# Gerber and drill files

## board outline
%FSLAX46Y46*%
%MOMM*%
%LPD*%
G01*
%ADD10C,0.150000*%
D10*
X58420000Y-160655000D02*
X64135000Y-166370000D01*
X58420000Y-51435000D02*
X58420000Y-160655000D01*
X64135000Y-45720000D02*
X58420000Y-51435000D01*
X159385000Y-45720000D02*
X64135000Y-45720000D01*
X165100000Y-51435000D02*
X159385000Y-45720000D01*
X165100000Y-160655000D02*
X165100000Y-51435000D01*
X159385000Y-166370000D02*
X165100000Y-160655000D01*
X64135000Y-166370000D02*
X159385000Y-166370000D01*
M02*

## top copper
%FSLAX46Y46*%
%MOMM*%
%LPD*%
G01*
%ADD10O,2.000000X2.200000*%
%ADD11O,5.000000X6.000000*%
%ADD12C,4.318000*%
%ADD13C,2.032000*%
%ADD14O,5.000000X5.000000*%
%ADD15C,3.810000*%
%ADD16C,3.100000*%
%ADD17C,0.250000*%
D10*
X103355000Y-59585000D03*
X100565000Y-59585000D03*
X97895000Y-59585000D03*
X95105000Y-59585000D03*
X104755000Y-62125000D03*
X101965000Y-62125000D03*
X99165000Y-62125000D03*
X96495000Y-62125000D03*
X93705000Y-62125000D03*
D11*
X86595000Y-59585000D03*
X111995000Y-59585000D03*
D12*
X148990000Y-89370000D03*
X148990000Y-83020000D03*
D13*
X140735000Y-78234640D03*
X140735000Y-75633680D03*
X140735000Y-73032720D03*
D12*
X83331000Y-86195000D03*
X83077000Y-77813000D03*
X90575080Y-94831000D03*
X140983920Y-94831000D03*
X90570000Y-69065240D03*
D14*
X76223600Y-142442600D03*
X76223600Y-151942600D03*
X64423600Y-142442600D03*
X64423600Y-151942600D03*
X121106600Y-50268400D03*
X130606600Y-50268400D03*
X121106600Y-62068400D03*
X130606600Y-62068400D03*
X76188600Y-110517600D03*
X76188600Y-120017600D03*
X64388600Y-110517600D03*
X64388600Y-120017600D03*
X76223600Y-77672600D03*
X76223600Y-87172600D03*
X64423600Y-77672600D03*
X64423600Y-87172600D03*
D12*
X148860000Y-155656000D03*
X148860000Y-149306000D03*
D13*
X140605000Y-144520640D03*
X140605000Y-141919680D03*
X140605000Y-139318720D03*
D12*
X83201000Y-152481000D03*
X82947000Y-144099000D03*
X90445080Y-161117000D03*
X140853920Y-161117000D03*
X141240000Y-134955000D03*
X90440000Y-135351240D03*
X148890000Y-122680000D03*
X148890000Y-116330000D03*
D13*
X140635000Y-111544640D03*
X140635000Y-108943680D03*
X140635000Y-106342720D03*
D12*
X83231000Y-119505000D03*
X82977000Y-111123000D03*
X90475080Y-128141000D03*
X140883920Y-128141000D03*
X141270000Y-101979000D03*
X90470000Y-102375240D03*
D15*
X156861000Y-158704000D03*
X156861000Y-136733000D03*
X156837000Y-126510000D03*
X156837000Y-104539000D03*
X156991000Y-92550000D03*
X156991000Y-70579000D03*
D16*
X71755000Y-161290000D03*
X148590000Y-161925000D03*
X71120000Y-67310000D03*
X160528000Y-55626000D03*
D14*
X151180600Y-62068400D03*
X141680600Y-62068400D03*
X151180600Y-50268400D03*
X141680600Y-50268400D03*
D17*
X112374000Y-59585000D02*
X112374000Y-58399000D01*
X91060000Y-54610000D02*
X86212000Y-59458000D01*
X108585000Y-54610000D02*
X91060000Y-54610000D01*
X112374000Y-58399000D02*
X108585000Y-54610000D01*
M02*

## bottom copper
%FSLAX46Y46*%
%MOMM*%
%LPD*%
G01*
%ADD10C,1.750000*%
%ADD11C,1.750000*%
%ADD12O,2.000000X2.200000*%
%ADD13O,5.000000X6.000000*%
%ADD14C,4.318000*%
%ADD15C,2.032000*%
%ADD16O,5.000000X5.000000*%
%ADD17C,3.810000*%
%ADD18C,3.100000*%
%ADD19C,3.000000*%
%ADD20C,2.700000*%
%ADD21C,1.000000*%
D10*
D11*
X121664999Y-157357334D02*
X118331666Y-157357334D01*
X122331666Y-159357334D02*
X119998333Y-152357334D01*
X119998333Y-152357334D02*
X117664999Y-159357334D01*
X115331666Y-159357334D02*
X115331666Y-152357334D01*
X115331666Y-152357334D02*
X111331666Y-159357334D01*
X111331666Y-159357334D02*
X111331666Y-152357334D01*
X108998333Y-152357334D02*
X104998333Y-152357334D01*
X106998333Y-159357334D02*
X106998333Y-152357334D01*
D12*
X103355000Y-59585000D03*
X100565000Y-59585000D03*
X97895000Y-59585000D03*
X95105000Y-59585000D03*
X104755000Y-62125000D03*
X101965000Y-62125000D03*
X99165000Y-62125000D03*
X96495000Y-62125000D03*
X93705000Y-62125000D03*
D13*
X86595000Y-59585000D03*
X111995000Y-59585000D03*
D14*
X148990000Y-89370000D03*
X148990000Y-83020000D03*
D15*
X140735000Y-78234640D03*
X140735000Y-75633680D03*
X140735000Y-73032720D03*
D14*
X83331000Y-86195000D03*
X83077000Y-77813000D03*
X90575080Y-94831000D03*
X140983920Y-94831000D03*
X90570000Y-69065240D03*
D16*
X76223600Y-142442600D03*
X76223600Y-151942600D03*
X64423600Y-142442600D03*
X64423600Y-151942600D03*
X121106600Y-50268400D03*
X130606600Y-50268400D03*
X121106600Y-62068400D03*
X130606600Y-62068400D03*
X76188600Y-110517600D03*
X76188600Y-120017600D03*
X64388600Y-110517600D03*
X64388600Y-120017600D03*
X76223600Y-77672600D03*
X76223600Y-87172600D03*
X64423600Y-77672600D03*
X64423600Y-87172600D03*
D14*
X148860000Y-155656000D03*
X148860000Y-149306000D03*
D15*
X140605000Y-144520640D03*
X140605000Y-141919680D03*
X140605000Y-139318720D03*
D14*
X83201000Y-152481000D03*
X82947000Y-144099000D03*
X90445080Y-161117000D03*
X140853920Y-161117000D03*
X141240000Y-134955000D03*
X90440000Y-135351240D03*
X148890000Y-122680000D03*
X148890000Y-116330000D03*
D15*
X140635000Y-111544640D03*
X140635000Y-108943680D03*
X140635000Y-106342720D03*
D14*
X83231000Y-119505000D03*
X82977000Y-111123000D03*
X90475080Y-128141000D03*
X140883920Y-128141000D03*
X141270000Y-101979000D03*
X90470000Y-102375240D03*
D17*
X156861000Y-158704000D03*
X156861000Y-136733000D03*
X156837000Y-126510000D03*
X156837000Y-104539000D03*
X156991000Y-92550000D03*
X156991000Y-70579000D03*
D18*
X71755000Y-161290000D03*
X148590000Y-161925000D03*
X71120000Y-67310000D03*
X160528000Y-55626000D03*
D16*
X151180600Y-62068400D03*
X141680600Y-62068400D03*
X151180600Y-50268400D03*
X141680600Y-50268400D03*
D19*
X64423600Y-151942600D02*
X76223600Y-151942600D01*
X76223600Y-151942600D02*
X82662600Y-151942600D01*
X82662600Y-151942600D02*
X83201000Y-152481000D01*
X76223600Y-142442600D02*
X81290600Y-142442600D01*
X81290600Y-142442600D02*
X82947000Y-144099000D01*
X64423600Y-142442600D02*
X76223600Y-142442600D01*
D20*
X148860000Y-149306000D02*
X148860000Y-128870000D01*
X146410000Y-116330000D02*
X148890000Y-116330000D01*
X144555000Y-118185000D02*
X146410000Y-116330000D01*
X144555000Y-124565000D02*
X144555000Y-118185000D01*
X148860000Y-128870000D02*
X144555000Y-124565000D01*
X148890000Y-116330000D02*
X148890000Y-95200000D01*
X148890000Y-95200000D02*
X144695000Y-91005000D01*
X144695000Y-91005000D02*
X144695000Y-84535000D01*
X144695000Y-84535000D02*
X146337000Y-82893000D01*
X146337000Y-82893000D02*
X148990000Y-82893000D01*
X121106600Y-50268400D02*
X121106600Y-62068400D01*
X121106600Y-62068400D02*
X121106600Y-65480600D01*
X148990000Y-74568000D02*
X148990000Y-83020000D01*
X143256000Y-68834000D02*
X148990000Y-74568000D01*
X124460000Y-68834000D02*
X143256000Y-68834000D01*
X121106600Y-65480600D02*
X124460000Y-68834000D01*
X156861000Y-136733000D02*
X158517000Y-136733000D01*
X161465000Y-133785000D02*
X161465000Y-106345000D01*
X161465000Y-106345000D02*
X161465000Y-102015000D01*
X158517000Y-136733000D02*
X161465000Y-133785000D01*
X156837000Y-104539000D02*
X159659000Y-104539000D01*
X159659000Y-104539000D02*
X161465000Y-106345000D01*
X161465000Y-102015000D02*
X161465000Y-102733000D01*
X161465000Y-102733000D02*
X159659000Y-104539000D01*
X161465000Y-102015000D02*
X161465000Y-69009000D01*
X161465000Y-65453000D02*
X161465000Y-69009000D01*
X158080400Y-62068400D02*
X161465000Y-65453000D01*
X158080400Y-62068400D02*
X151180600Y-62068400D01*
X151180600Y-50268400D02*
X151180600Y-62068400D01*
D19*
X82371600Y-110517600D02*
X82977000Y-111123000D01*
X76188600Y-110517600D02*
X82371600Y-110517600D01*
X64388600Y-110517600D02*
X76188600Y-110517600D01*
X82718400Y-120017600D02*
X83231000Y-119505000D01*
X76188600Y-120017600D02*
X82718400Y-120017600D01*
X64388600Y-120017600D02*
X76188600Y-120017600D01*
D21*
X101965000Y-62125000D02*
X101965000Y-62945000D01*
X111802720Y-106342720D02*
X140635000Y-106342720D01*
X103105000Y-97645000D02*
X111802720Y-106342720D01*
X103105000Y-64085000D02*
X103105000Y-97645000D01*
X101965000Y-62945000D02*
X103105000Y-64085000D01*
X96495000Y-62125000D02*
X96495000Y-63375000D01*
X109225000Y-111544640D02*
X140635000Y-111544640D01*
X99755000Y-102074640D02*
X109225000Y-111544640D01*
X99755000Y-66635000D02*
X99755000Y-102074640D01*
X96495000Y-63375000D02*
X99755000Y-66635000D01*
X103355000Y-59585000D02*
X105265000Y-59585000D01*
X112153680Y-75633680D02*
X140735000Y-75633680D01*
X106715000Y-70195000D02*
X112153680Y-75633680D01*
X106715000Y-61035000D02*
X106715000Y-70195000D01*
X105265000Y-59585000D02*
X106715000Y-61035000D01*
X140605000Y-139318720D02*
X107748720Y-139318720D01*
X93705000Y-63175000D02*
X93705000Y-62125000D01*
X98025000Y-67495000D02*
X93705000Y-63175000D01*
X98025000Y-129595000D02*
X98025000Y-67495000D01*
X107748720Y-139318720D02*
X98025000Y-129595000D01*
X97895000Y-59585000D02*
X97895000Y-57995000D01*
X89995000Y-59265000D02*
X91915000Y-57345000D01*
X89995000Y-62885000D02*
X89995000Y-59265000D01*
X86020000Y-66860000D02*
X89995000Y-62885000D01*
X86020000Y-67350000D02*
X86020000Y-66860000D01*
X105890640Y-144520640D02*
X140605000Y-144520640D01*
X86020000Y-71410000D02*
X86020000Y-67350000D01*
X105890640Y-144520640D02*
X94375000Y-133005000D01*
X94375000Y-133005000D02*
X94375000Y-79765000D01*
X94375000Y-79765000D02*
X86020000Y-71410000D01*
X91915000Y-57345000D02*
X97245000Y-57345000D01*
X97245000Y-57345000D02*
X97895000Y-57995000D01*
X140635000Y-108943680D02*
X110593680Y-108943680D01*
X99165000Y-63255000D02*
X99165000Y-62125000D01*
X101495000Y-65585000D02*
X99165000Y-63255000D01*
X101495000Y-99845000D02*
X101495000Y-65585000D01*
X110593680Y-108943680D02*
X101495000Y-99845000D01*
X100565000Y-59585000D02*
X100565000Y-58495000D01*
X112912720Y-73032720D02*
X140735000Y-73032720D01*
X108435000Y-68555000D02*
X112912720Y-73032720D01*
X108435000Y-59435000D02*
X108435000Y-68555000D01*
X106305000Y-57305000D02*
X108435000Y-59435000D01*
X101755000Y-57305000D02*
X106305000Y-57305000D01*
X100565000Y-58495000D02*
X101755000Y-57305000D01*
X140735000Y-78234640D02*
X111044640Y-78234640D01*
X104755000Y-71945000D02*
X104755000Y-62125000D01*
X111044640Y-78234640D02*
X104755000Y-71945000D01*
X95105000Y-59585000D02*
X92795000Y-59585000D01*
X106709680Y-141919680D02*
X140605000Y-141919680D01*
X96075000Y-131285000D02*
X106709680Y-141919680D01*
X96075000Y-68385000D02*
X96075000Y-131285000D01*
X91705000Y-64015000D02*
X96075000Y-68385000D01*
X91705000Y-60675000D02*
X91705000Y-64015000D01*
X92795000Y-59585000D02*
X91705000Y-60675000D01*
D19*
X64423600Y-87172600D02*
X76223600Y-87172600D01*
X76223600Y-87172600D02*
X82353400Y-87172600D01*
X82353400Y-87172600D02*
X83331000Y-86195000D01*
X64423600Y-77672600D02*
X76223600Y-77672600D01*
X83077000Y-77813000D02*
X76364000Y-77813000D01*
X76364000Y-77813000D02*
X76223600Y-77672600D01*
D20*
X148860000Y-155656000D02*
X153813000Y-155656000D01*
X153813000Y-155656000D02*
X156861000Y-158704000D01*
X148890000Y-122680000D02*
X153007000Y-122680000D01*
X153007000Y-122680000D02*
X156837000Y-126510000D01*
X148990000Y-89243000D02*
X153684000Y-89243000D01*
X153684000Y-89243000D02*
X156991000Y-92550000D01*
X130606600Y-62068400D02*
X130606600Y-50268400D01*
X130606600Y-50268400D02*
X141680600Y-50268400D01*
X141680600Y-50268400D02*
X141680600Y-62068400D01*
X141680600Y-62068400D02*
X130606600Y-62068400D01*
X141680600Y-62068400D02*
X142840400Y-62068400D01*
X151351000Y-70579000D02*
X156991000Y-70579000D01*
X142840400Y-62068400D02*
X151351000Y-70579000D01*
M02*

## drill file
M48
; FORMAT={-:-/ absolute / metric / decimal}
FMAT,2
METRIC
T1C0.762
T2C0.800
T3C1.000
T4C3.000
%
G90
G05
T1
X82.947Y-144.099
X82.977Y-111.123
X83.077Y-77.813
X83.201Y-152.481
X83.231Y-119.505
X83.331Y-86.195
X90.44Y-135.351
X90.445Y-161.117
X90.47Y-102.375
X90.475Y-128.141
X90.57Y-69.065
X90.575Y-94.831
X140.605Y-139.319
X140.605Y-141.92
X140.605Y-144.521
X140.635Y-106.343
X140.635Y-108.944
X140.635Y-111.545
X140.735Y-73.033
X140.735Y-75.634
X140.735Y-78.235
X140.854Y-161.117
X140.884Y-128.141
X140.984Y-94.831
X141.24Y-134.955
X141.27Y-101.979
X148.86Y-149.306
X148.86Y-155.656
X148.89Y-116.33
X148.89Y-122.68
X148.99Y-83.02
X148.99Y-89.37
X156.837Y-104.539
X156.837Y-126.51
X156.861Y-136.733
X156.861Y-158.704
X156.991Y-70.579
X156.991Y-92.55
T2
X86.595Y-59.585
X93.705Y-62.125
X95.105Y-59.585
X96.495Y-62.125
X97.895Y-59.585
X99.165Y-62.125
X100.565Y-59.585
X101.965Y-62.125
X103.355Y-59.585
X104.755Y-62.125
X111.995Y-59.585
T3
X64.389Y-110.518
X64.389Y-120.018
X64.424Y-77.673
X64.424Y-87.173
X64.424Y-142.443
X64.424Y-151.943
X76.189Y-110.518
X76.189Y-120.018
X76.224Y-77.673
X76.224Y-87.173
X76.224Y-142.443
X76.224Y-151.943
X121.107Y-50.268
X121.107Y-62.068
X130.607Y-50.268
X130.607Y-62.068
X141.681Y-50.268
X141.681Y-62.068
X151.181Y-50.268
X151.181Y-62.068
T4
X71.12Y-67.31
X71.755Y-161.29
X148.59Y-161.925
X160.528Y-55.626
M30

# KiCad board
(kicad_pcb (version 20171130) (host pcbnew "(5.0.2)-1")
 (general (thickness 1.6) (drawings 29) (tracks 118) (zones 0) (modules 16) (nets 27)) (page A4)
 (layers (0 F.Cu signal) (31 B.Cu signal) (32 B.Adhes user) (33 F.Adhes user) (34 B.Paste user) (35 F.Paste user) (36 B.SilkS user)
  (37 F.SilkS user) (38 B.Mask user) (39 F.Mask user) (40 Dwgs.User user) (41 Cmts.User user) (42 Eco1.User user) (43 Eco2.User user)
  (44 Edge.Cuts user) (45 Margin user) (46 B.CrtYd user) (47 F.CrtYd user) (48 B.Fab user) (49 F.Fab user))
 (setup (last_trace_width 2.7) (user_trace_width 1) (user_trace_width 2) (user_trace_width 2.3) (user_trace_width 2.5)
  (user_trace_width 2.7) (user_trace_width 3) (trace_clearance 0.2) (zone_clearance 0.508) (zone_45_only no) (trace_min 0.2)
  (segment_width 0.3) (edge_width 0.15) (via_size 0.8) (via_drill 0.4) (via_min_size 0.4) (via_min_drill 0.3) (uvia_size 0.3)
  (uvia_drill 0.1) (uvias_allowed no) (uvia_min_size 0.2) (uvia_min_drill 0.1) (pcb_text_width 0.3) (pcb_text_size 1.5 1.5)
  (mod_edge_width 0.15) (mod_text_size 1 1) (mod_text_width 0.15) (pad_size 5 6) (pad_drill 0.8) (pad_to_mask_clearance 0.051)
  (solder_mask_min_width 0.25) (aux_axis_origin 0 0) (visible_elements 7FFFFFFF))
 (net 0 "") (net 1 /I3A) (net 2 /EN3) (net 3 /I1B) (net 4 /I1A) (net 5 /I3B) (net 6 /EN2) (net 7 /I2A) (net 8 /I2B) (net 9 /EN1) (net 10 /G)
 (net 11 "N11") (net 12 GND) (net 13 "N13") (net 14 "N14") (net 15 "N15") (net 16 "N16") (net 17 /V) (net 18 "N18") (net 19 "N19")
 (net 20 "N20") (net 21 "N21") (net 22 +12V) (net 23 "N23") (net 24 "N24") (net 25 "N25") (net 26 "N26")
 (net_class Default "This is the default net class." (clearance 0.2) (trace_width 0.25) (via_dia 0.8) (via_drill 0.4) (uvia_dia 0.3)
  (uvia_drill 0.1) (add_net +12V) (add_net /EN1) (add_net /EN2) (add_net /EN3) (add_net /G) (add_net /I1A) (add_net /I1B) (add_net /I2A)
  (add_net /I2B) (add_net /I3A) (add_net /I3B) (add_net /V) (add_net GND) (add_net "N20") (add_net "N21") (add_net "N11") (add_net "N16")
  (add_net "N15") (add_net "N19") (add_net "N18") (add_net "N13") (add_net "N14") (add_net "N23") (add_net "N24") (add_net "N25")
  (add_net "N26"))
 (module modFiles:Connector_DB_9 (layer F.Cu) (at 93.705 62.125)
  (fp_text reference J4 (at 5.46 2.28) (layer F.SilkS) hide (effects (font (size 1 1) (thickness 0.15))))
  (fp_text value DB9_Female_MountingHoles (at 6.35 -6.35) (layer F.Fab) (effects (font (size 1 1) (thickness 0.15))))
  (pad 9 thru_hole oval (at 9.65 -2.54) (size 2 2.2) (drill 0.8) (layers *.Cu *.Mask) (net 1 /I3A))
  (pad 8 thru_hole oval (at 6.86 -2.54) (size 2 2.2) (drill 0.8) (layers *.Cu *.Mask) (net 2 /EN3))
  (pad 7 thru_hole oval (at 4.19 -2.54) (size 2 2.2) (drill 0.8) (layers *.Cu *.Mask) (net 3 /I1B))
  (pad 6 thru_hole oval (at 1.4 -2.54) (size 2 2.2) (drill 0.8) (layers *.Cu *.Mask) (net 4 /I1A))
  (pad 5 thru_hole oval (at 11.05 0) (size 2 2.2) (drill 0.8) (layers *.Cu *.Mask) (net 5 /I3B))
  (pad 4 thru_hole oval (at 8.26 0) (size 2 2.2) (drill 0.8) (layers *.Cu *.Mask) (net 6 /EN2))
  (pad 3 thru_hole oval (at 5.46 0) (size 2 2.2) (drill 0.8) (layers *.Cu *.Mask) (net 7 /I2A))
  (pad 2 thru_hole oval (at 2.79 0) (size 2 2.2) (drill 0.8) (layers *.Cu *.Mask) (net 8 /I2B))
  (pad 1 thru_hole oval (at 0 0) (size 2 2.2) (drill 0.8) (layers *.Cu *.Mask) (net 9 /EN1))
  (pad 0 thru_hole oval (at -7.11 -2.54) (size 5 6) (drill 0.8) (layers *.Cu *.Mask) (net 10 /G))
  (pad 0 thru_hole oval (at 18.29 -2.54) (size 5 6) (drill 0.8) (layers *.Cu *.Mask) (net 10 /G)))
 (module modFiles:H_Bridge (layer F.Cu) (at 139.465 83.655)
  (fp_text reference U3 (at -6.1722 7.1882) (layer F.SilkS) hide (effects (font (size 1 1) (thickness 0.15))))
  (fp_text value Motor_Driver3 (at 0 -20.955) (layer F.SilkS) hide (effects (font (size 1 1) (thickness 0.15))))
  (pad 6 thru_hole circle (at 9.525 5.715) (size 4.318 4.318) (drill 0.762) (layers *.Cu *.Mask F.SilkS) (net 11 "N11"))
  (pad 7 thru_hole circle (at 9.525 -0.635) (size 4.318 4.318) (drill 0.762) (layers *.Cu *.Mask F.SilkS) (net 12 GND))
  (pad 5 thru_hole circle (at 1.27 -5.42036) (size 2.032 2.032) (drill 0.762) (layers *.Cu *.Mask F.SilkS) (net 5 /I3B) (clearance -0.254))
  (pad 4 thru_hole circle (at 1.27 -8.02132) (size 2.032 2.032) (drill 0.762) (layers *.Cu *.Mask F.SilkS) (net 1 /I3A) (clearance -0.254))
  (pad 3 thru_hole circle (at 1.27 -10.62228) (size 2.032 2.032) (drill 0.762) (layers *.Cu *.Mask F.SilkS) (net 2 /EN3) (clearance -0.254))
  (pad 1 thru_hole circle (at -56.134 2.54) (size 4.318 4.318) (drill 0.762) (layers *.Cu *.Mask F.SilkS) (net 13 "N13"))
  (pad 2 thru_hole circle (at -56.388 -5.842) (size 4.318 4.318) (drill 0.762) (layers *.Cu *.Mask F.SilkS) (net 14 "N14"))
  (pad "" thru_hole circle (at -48.88992 11.176) (size 4.318 4.318) (drill 0.762) (layers *.Cu *.Mask F.SilkS))
  (pad "" thru_hole circle (at 1.51892 11.176) (size 4.318 4.318) (drill 0.762) (layers *.Cu *.Mask F.SilkS))
  (pad "" thru_hole circle (at -48.895 -14.58976) (size 4.318 4.318) (drill 0.762) (layers *.Cu *.Mask F.SilkS)))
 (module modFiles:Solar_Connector (layer F.Cu) (at 69.85 147.32 90)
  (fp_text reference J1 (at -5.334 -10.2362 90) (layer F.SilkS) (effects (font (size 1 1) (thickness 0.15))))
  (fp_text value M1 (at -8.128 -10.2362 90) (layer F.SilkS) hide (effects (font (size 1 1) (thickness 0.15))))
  (pad 2 thru_hole oval (at 4.8774 6.3736 180) (size 5 5) (drill 1) (layers *.Cu *.Mask F.SilkS) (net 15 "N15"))
  (pad 1 thru_hole oval (at -4.6226 6.3736 180) (size 5 5) (drill 1) (layers *.Cu *.Mask F.SilkS) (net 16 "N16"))
  (pad 2 thru_hole oval (at 4.8774 -5.4264 180) (size 5 5) (drill 1) (layers *.Cu *.Mask F.SilkS) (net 15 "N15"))
  (pad 1 thru_hole oval (at -4.6226 -5.4264 180) (size 5 5) (drill 1) (layers *.Cu *.Mask F.SilkS) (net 16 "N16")))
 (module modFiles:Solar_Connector (layer F.Cu) (at 125.984 56.642 180)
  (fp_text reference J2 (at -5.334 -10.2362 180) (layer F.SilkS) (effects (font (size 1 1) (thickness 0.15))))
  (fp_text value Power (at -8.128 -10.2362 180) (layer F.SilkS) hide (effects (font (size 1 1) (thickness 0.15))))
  (pad 2 thru_hole oval (at 4.8774 6.3736 270) (size 5 5) (drill 1) (layers *.Cu *.Mask F.SilkS) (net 12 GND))
  (pad 1 thru_hole oval (at -4.6226 6.3736 270) (size 5 5) (drill 1) (layers *.Cu *.Mask F.SilkS) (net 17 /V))
  (pad 2 thru_hole oval (at 4.8774 -5.4264 270) (size 5 5) (drill 1) (layers *.Cu *.Mask F.SilkS) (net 12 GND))
  (pad 1 thru_hole oval (at -4.6226 -5.4264 270) (size 5 5) (drill 1) (layers *.Cu *.Mask F.SilkS) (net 17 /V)))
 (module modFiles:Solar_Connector (layer F.Cu) (at 69.815 115.395 90)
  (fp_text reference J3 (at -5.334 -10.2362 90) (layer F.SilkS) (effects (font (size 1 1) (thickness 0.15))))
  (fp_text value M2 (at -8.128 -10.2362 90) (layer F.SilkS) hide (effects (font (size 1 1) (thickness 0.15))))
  (pad 2 thru_hole oval (at 4.8774 6.3736 180) (size 5 5) (drill 1) (layers *.Cu *.Mask F.SilkS) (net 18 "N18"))
  (pad 1 thru_hole oval (at -4.6226 6.3736 180) (size 5 5) (drill 1) (layers *.Cu *.Mask F.SilkS) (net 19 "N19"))
  (pad 2 thru_hole oval (at 4.8774 -5.4264 180) (size 5 5) (drill 1) (layers *.Cu *.Mask F.SilkS) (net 18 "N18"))
  (pad 1 thru_hole oval (at -4.6226 -5.4264 180) (size 5 5) (drill 1) (layers *.Cu *.Mask F.SilkS) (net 19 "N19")))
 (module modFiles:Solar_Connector (layer F.Cu) (at 69.85 82.55 90)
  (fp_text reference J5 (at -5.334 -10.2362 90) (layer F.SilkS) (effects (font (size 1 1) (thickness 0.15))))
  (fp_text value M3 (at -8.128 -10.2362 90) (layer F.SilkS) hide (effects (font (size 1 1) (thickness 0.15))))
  (pad 2 thru_hole oval (at 4.8774 6.3736 180) (size 5 5) (drill 1) (layers *.Cu *.Mask F.SilkS) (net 14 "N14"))
  (pad 1 thru_hole oval (at -4.6226 6.3736 180) (size 5 5) (drill 1) (layers *.Cu *.Mask F.SilkS) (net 13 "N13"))
  (pad 2 thru_hole oval (at 4.8774 -5.4264 180) (size 5 5) (drill 1) (layers *.Cu *.Mask F.SilkS) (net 14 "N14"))
  (pad 1 thru_hole oval (at -4.6226 -5.4264 180) (size 5 5) (drill 1) (layers *.Cu *.Mask F.SilkS) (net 13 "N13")))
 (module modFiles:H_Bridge (layer F.Cu) (at 139.335 149.941)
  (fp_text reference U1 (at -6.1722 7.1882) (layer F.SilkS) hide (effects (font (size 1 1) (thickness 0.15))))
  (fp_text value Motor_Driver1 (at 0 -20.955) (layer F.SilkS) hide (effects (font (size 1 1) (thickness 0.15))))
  (pad 6 thru_hole circle (at 9.525 5.715) (size 4.318 4.318) (drill 0.762) (layers *.Cu *.Mask F.SilkS) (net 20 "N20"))
  (pad 7 thru_hole circle (at 9.525 -0.635) (size 4.318 4.318) (drill 0.762) (layers *.Cu *.Mask F.SilkS) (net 12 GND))
  (pad 5 thru_hole circle (at 1.27 -5.42036) (size 2.032 2.032) (drill 0.762) (layers *.Cu *.Mask F.SilkS) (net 3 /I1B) (clearance -0.254))
  (pad 4 thru_hole circle (at 1.27 -8.02132) (size 2.032 2.032) (drill 0.762) (layers *.Cu *.Mask F.SilkS) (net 4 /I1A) (clearance -0.254))
  (pad 3 thru_hole circle (at 1.27 -10.62228) (size 2.032 2.032) (drill 0.762) (layers *.Cu *.Mask F.SilkS) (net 9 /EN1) (clearance -0.254))
  (pad 1 thru_hole circle (at -56.134 2.54) (size 4.318 4.318) (drill 0.762) (layers *.Cu *.Mask F.SilkS) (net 16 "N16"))
  (pad 2 thru_hole circle (at -56.388 -5.842) (size 4.318 4.318) (drill 0.762) (layers *.Cu *.Mask F.SilkS) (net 15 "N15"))
  (pad "" thru_hole circle (at -48.88992 11.176) (size 4.318 4.318) (drill 0.762) (layers *.Cu *.Mask F.SilkS))
  (pad "" thru_hole circle (at 1.51892 11.176) (size 4.318 4.318) (drill 0.762) (layers *.Cu *.Mask F.SilkS))
  (pad "" thru_hole circle (at 1.905 -14.986) (size 4.318 4.318) (drill 0.762) (layers *.Cu *.Mask F.SilkS))
  (pad "" thru_hole circle (at -48.895 -14.58976) (size 4.318 4.318) (drill 0.762) (layers *.Cu *.Mask F.SilkS)))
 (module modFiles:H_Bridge (layer F.Cu) (at 139.365 116.965)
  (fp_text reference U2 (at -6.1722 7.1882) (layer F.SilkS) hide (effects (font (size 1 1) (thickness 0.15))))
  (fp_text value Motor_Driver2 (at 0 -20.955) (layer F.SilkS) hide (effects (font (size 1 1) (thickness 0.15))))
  (pad 6 thru_hole circle (at 9.525 5.715) (size 4.318 4.318) (drill 0.762) (layers *.Cu *.Mask F.SilkS) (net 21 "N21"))
  (pad 7 thru_hole circle (at 9.525 -0.635) (size 4.318 4.318) (drill 0.762) (layers *.Cu *.Mask F.SilkS) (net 12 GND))
  (pad 5 thru_hole circle (at 1.27 -5.42036) (size 2.032 2.032) (drill 0.762) (layers *.Cu *.Mask F.SilkS) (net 8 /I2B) (clearance -0.254))
  (pad 4 thru_hole circle (at 1.27 -8.02132) (size 2.032 2.032) (drill 0.762) (layers *.Cu *.Mask F.SilkS) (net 7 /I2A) (clearance -0.254))
  (pad 3 thru_hole circle (at 1.27 -10.62228) (size 2.032 2.032) (drill 0.762) (layers *.Cu *.Mask F.SilkS) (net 6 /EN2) (clearance -0.254))
  (pad 1 thru_hole circle (at -56.134 2.54) (size 4.318 4.318) (drill 0.762) (layers *.Cu *.Mask F.SilkS) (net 19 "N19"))
  (pad 2 thru_hole circle (at -56.388 -5.842) (size 4.318 4.318) (drill 0.762) (layers *.Cu *.Mask F.SilkS) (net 18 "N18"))
  (pad "" thru_hole circle (at -48.88992 11.176) (size 4.318 4.318) (drill 0.762) (layers *.Cu *.Mask F.SilkS))
  (pad "" thru_hole circle (at 1.51892 11.176) (size 4.318 4.318) (drill 0.762) (layers *.Cu *.Mask F.SilkS))
  (pad "" thru_hole circle (at 1.905 -14.986) (size 4.318 4.318) (drill 0.762) (layers *.Cu *.Mask F.SilkS))
  (pad "" thru_hole circle (at -48.895 -14.58976) (size 4.318 4.318) (drill 0.762) (layers *.Cu *.Mask F.SilkS)))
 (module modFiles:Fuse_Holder (layer F.Cu) (at 157.369 147.909 90)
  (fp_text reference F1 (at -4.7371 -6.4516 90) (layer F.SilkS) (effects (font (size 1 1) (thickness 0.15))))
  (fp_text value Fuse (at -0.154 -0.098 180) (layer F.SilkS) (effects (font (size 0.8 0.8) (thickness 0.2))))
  (pad 2 thru_hole circle (at -10.795 -0.508 180) (size 3.81 3.81) (drill 0.762) (layers *.Cu *.Mask F.SilkS) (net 20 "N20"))
  (pad 1 thru_hole circle (at 11.176 -0.508 180) (size 3.81 3.81) (drill 0.762) (layers *.Cu *.Mask F.SilkS) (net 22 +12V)))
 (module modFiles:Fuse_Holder (layer F.Cu) (at 157.345 115.715 90)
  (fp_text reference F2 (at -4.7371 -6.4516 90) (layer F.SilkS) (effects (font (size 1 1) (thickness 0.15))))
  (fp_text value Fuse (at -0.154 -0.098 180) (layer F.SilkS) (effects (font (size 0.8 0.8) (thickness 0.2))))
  (pad 2 thru_hole circle (at -10.795 -0.508 180) (size 3.81 3.81) (drill 0.762) (layers *.Cu *.Mask F.SilkS) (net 21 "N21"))
  (pad 1 thru_hole circle (at 11.176 -0.508 180) (size 3.81 3.81) (drill 0.762) (layers *.Cu *.Mask F.SilkS) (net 22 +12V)))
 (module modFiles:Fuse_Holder (layer F.Cu) (at 157.499 81.755 90)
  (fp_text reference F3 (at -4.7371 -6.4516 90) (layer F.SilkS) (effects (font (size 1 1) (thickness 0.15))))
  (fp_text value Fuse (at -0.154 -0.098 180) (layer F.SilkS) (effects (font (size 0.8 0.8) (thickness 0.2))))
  (pad 2 thru_hole circle (at -10.795 -0.508 180) (size 3.81 3.81) (drill 0.762) (layers *.Cu *.Mask F.SilkS) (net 11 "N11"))
  (pad 1 thru_hole circle (at 11.176 -0.508 180) (size 3.81 3.81) (drill 0.762) (layers *.Cu *.Mask F.SilkS) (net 17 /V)))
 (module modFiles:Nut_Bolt (layer F.Cu) (at 71.755 161.29 90)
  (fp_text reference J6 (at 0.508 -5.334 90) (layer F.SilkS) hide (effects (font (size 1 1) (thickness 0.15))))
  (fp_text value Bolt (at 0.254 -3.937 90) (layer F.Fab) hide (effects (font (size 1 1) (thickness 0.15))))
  (pad 1 thru_hole circle (at 0 0 90) (size 3.1 3.1) (drill 3) (layers *.Cu *.Mask) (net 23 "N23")))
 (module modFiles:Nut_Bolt (layer F.Cu) (at 148.59 161.925 90)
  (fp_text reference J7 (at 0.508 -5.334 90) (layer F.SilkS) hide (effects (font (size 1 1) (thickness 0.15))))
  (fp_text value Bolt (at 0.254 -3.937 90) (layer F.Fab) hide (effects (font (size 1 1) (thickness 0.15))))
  (pad 1 thru_hole circle (at 0 0 90) (size 3.1 3.1) (drill 3) (layers *.Cu *.Mask) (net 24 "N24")))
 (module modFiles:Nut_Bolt (layer F.Cu) (at 71.12 67.31 90)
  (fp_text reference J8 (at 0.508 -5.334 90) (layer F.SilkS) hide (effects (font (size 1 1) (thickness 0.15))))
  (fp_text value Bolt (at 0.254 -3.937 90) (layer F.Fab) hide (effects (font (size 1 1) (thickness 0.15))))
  (pad 1 thru_hole circle (at 0 0 90) (size 3.1 3.1) (drill 3) (layers *.Cu *.Mask) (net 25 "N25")))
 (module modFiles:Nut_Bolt (layer F.Cu) (at 160.528 55.626 90)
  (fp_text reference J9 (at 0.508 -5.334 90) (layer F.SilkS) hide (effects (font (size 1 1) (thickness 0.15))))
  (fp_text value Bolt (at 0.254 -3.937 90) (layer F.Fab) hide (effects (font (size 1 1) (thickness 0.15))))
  (pad 1 thru_hole circle (at 0 0 90) (size 3.1 3.1) (drill 3) (layers *.Cu *.Mask) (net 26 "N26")))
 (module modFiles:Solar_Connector (layer F.Cu) (at 146.558 56.642 180)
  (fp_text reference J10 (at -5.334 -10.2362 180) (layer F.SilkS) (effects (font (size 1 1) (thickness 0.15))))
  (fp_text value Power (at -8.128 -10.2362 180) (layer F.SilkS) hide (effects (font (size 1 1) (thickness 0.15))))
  (pad 1 thru_hole oval (at -4.6226 -5.4264 270) (size 5 5) (drill 1) (layers *.Cu *.Mask F.SilkS) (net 22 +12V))
  (pad 2 thru_hole oval (at 4.8774 -5.4264 270) (size 5 5) (drill 1) (layers *.Cu *.Mask F.SilkS) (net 17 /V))
  (pad 1 thru_hole oval (at -4.6226 6.3736 270) (size 5 5) (drill 1) (layers *.Cu *.Mask F.SilkS) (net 22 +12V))
  (pad 2 thru_hole oval (at 4.8774 6.3736 270) (size 5 5) (drill 1) (layers *.Cu *.Mask F.SilkS) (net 17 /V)))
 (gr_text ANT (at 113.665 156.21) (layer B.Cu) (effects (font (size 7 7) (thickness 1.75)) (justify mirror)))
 (gr_line (start 58.42 160.655) (end 64.135 166.37) (angle 90) (layer Edge.Cuts) (width 0.15))
 (gr_line (start 58.42 51.435) (end 58.42 160.655) (angle 90) (layer Edge.Cuts) (width 0.15))
 (gr_line (start 64.135 45.72) (end 58.42 51.435) (angle 90) (layer Edge.Cuts) (width 0.15))
 (gr_line (start 159.385 45.72) (end 64.135 45.72) (angle 90) (layer Edge.Cuts) (width 0.15))
 (gr_line (start 165.1 51.435) (end 159.385 45.72) (angle 90) (layer Edge.Cuts) (width 0.15))
 (gr_line (start 165.1 160.655) (end 165.1 51.435) (angle 90) (layer Edge.Cuts) (width 0.15))
 (gr_line (start 159.385 166.37) (end 165.1 160.655) (angle 90) (layer Edge.Cuts) (width 0.15))
 (gr_line (start 64.135 166.37) (end 159.385 166.37) (angle 90) (layer Edge.Cuts) (width 0.15))
 (segment (start 112.374 59.585) (end 112.374 58.399) (width 0.25) (layer F.Cu) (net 10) (status C00030))
 (segment (start 91.06 54.61) (end 86.212 59.458) (width 0.25) (layer F.Cu) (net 10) (status 800020))
 (segment (start 108.585 54.61) (end 91.06 54.61) (width 0.25) (layer F.Cu) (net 10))
 (segment (start 112.374 58.399) (end 108.585 54.61) (width 0.25) (layer F.Cu) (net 10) (status 400010))
 (segment (start 64.4236 151.9426) (end 76.2236 151.9426) (width 3) (layer B.Cu) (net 16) (status C00030))
 (segment (start 76.2236 151.9426) (end 82.6626 151.9426) (width 3) (layer B.Cu) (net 16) (status C00030))
 (segment (start 82.6626 151.9426) (end 83.201 152.481) (width 3) (layer B.Cu) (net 16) (status C00030))
 (segment (start 76.2236 142.4426) (end 81.2906 142.4426) (width 3) (layer B.Cu) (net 15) (status 400010))
 (segment (start 81.2906 142.4426) (end 82.947 144.099) (width 3) (layer B.Cu) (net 15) (status 800020))
 (segment (start 64.4236 142.4426) (end 76.2236 142.4426) (width 3) (layer B.Cu) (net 15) (status C00030))
 (segment (start 148.86 149.306) (end 148.86 128.87) (width 2.7) (layer B.Cu) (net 12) (status 400010))
 (segment (start 146.41 116.33) (end 148.89 116.33) (width 2.7) (layer B.Cu) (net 12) (status 800020))
 (segment (start 144.555 118.185) (end 146.41 116.33) (width 2.7) (layer B.Cu) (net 12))
 (segment (start 144.555 124.565) (end 144.555 118.185) (width 2.7) (layer B.Cu) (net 12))
 (segment (start 148.86 128.87) (end 144.555 124.565) (width 2.7) (layer B.Cu) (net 12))
 (segment (start 148.89 116.33) (end 148.89 95.2) (width 2.7) (layer B.Cu) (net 12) (status 400010))
 (segment (start 148.89 95.2) (end 144.695 91.005) (width 2.7) (layer B.Cu) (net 12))
 (segment (start 144.695 91.005) (end 144.695 84.535) (width 2.7) (layer B.Cu) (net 12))
 (segment (start 144.695 84.535) (end 146.337 82.893) (width 2.7) (layer B.Cu) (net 12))
 (segment (start 146.337 82.893) (end 148.99 82.893) (width 2.7) (layer B.Cu) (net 12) (status 800020))
 (segment (start 121.1066 50.2684) (end 121.1066 62.0684) (width 2.7) (layer B.Cu) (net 12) (status C00030))
 (segment (start 121.1066 62.0684) (end 121.1066 65.4806) (width 2.7) (layer B.Cu) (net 12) (status 400010))
 (segment (start 148.99 74.568) (end 148.99 83.02) (width 2.7) (layer B.Cu) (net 12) (status 800020))
 (segment (start 143.256 68.834) (end 148.99 74.568) (width 2.7) (layer B.Cu) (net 12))
 (segment (start 124.46 68.834) (end 143.256 68.834) (width 2.7) (layer B.Cu) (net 12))
 (segment (start 121.1066 65.4806) (end 124.46 68.834) (width 2.7) (layer B.Cu) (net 12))
 (segment (start 156.861 136.733) (end 158.517 136.733) (width 2.7) (layer B.Cu) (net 22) (status C00030))
 (segment (start 161.465 133.785) (end 161.465 106.345) (width 2.7) (layer B.Cu) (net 22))
 (segment (start 161.465 106.345) (end 161.465 102.015) (width 2.7) (layer B.Cu) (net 22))
 (segment (start 158.517 136.733) (end 161.465 133.785) (width 2.7) (layer B.Cu) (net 22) (status 400010))
 (segment (start 156.837 104.539) (end 159.659 104.539) (width 2.7) (layer B.Cu) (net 22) (status 400010))
 (segment (start 159.659 104.539) (end 161.465 106.345) (width 2.7) (layer B.Cu) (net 22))
 (segment (start 161.465 102.015) (end 161.465 102.733) (width 2.7) (layer B.Cu) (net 22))
 (segment (start 161.465 102.733) (end 159.659 104.539) (width 2.7) (layer B.Cu) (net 22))
 (segment (start 161.465 102.015) (end 161.465 69.009) (width 2.7) (layer B.Cu) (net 22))
 (segment (start 161.465 65.453) (end 161.465 69.009) (width 2.7) (layer B.Cu) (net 22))
 (segment (start 158.0804 62.0684) (end 161.465 65.453) (width 2.7) (layer B.Cu) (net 22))
 (segment (start 158.0804 62.0684) (end 151.1806 62.0684) (width 2.7) (layer B.Cu) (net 22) (status 800000))
 (segment (start 151.1806 50.2684) (end 151.1806 62.0684) (width 2.7) (layer B.Cu) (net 22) (status C00000))
 (segment (start 82.3716 110.5176) (end 82.977 111.123) (width 3) (layer B.Cu) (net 18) (status C00030))
 (segment (start 76.1886 110.5176) (end 82.3716 110.5176) (width 3) (layer B.Cu) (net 18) (status C00030))
 (segment (start 64.3886 110.5176) (end 76.1886 110.5176) (width 3) (layer B.Cu) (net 18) (status C00030))
 (segment (start 82.7184 120.0176) (end 83.231 119.505) (width 3) (layer B.Cu) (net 19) (status C00030))
 (segment (start 76.1886 120.0176) (end 82.7184 120.0176) (width 3) (layer B.Cu) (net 19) (status C00030))
 (segment (start 64.3886 120.0176) (end 76.1886 120.0176) (width 3) (layer B.Cu) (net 19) (status C00030))
 (segment (start 101.965 62.125) (end 101.965 62.945) (width 1) (layer B.Cu) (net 6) (status 400030))
 (segment (start 111.80272 106.34272) (end 140.635 106.34272) (width 1) (layer B.Cu) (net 6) (status 800020))
 (segment (start 103.105 97.645) (end 111.80272 106.34272) (width 1) (layer B.Cu) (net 6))
 (segment (start 103.105 64.085) (end 103.105 97.645) (width 1) (layer B.Cu) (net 6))
 (segment (start 101.965 62.945) (end 103.105 64.085) (width 1) (layer B.Cu) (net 6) (status 10))
 (segment (start 96.495 62.125) (end 96.495 63.375) (width 1) (layer B.Cu) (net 8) (status 400010))
 (segment (start 109.225 111.54464) (end 140.635 111.54464) (width 1) (layer B.Cu) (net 8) (status 800020))
 (segment (start 99.755 102.07464) (end 109.225 111.54464) (width 1) (layer B.Cu) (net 8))
 (segment (start 99.755 66.635) (end 99.755 102.07464) (width 1) (layer B.Cu) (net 8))
 (segment (start 96.495 63.375) (end 99.755 66.635) (width 1) (layer B.Cu) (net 8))
 (segment (start 103.355 59.585) (end 105.265 59.585) (width 1) (layer B.Cu) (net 1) (status 400010))
 (segment (start 112.15368 75.63368) (end 140.735 75.63368) (width 1) (layer B.Cu) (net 1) (status 800020))
 (segment (start 106.715 70.195) (end 112.15368 75.63368) (width 1) (layer B.Cu) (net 1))
 (segment (start 106.715 61.035) (end 106.715 70.195) (width 1) (layer B.Cu) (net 1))
 (segment (start 105.265 59.585) (end 106.715 61.035) (width 1) (layer B.Cu) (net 1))
 (segment (start 140.605 139.31872) (end 107.74872 139.31872) (width 1) (layer B.Cu) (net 9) (status 400010))
 (segment (start 93.705 63.175) (end 93.705 62.125) (width 1) (layer B.Cu) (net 9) (status 800030))
 (segment (start 98.025 67.495) (end 93.705 63.175) (width 1) (layer B.Cu) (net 9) (status 20))
 (segment (start 98.025 129.595) (end 98.025 67.495) (width 1) (layer B.Cu) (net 9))
 (segment (start 107.74872 139.31872) (end 98.025 129.595) (width 1) (layer B.Cu) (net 9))
 (segment (start 97.895 59.585) (end 97.895 57.995) (width 1) (layer B.Cu) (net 3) (status 400010))
 (segment (start 89.995 59.265) (end 91.915 57.345) (width 1) (layer B.Cu) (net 3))
 (segment (start 89.995 62.885) (end 89.995 59.265) (width 1) (layer B.Cu) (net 3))
 (segment (start 86.02 66.86) (end 89.995 62.885) (width 1) (layer B.Cu) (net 3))
 (segment (start 86.02 67.35) (end 86.02 66.86) (width 1) (layer B.Cu) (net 3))
 (segment (start 105.89064 144.52064) (end 140.605 144.52064) (width 1) (layer B.Cu) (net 3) (status 800020))
 (segment (start 86.02 71.41) (end 86.02 67.35) (width 1) (layer B.Cu) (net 3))
 (segment (start 105.89064 144.52064) (end 94.375 133.005) (width 1) (layer B.Cu) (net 3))
 (segment (start 94.375 133.005) (end 94.375 79.765) (width 1) (layer B.Cu) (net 3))
 (segment (start 94.375 79.765) (end 86.02 71.41) (width 1) (layer B.Cu) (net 3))
 (segment (start 91.915 57.345) (end 97.245 57.345) (width 1) (layer B.Cu) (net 3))
 (segment (start 97.245 57.345) (end 97.895 57.995) (width 1) (layer B.Cu) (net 3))
 (segment (start 140.635 108.94368) (end 110.59368 108.94368) (width 1) (layer B.Cu) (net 7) (status 400010))
 (segment (start 99.165 63.255) (end 99.165 62.125) (width 1) (layer B.Cu) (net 7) (status 800020))
 (segment (start 101.495 65.585) (end 99.165 63.255) (width 1) (layer B.Cu) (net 7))
 (segment (start 101.495 99.845) (end 101.495 65.585) (width 1) (layer B.Cu) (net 7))
 (segment (start 110.59368 108.94368) (end 101.495 99.845) (width 1) (layer B.Cu) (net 7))
 (segment (start 100.565 59.585) (end 100.565 58.495) (width 1) (layer B.Cu) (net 2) (status 400030))
 (segment (start 112.91272 73.03272) (end 140.735 73.03272) (width 1) (layer B.Cu) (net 2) (status 800020))
 (segment (start 108.435 68.555) (end 112.91272 73.03272) (width 1) (layer B.Cu) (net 2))
 (segment (start 108.435 59.435) (end 108.435 68.555) (width 1) (layer B.Cu) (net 2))
 (segment (start 106.305 57.305) (end 108.435 59.435) (width 1) (layer B.Cu) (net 2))
 (segment (start 101.755 57.305) (end 106.305 57.305) (width 1) (layer B.Cu) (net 2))
 (segment (start 100.565 58.495) (end 101.755 57.305) (width 1) (layer B.Cu) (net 2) (status 10))
 (segment (start 140.735 78.23464) (end 111.04464 78.23464) (width 1) (layer B.Cu) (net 5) (status 400010))
 (segment (start 104.755 71.945) (end 104.755 62.125) (width 1) (layer B.Cu) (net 5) (status 800020))
 (segment (start 111.04464 78.23464) (end 104.755 71.945) (width 1) (layer B.Cu) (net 5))
 (segment (start 95.105 59.585) (end 92.795 59.585) (width 1) (layer B.Cu) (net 4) (status 400010))
 (segment (start 106.70968 141.91968) (end 140.605 141.91968) (width 1) (layer B.Cu) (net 4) (status 800020))
 (segment (start 96.075 131.285) (end 106.70968 141.91968) (width 1) (layer B.Cu) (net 4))
 (segment (start 96.075 68.385) (end 96.075 131.285) (width 1) (layer B.Cu) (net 4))
 (segment (start 91.705 64.015) (end 96.075 68.385) (width 1) (layer B.Cu) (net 4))
 (segment (start 91.705 60.675) (end 91.705 64.015) (width 1) (layer B.Cu) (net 4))
 (segment (start 92.795 59.585) (end 91.705 60.675) (width 1) (layer B.Cu) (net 4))
 (segment (start 64.4236 87.1726) (end 76.2236 87.1726) (width 3) (layer B.Cu) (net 13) (status C00030))
 (segment (start 76.2236 87.1726) (end 82.3534 87.1726) (width 3) (layer B.Cu) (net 13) (status C00030))
 (segment (start 82.3534 87.1726) (end 83.331 86.195) (width 3) (layer B.Cu) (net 13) (status C00030))
 (segment (start 64.4236 77.6726) (end 76.2236 77.6726) (width 3) (layer B.Cu) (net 14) (status C00030))
 (segment (start 83.077 77.813) (end 76.364 77.813) (width 3) (layer B.Cu) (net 14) (status C00030))
 (segment (start 76.364 77.813) (end 76.2236 77.6726) (width 3) (layer B.Cu) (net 14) (status C00030))
 (segment (start 148.86 155.656) (end 153.813 155.656) (width 2.7) (layer B.Cu) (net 20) (status 400010))
 (segment (start 153.813 155.656) (end 156.861 158.704) (width 2.7) (layer B.Cu) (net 20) (status 800020))
 (segment (start 148.89 122.68) (end 153.007 122.68) (width 2.7) (layer B.Cu) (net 21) (status 400010))
 (segment (start 153.007 122.68) (end 156.837 126.51) (width 2.7) (layer B.Cu) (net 21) (status 800020))
 (segment (start 148.99 89.243) (end 153.684 89.243) (width 2.7) (layer B.Cu) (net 11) (status 400010))
 (segment (start 153.684 89.243) (end 156.991 92.55) (width 2.7) (layer B.Cu) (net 11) (status 800020))
 (segment (start 130.6066 62.0684) (end 130.6066 50.2684) (width 2.7) (layer B.Cu) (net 17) (status C00030))
 (segment (start 130.6066 50.2684) (end 141.6806 50.2684) (width 2.7) (layer B.Cu) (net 17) (status C00030))
 (segment (start 141.6806 50.2684) (end 141.6806 62.0684) (width 2.7) (layer B.Cu) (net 17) (status C00030))
 (segment (start 141.6806 62.0684) (end 130.6066 62.0684) (width 2.7) (layer B.Cu) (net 17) (status C00030))
 (segment (start 141.6806 62.0684) (end 142.8404 62.0684) (width 2.7) (layer B.Cu) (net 17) (status C00000))
 (segment (start 151.351 70.579) (end 156.991 70.579) (width 2.7) (layer B.Cu) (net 17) (status 800000))
 (segment (start 142.8404 62.0684) (end 151.351 70.579) (width 2.7) (layer B.Cu) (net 17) (status 400000)))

